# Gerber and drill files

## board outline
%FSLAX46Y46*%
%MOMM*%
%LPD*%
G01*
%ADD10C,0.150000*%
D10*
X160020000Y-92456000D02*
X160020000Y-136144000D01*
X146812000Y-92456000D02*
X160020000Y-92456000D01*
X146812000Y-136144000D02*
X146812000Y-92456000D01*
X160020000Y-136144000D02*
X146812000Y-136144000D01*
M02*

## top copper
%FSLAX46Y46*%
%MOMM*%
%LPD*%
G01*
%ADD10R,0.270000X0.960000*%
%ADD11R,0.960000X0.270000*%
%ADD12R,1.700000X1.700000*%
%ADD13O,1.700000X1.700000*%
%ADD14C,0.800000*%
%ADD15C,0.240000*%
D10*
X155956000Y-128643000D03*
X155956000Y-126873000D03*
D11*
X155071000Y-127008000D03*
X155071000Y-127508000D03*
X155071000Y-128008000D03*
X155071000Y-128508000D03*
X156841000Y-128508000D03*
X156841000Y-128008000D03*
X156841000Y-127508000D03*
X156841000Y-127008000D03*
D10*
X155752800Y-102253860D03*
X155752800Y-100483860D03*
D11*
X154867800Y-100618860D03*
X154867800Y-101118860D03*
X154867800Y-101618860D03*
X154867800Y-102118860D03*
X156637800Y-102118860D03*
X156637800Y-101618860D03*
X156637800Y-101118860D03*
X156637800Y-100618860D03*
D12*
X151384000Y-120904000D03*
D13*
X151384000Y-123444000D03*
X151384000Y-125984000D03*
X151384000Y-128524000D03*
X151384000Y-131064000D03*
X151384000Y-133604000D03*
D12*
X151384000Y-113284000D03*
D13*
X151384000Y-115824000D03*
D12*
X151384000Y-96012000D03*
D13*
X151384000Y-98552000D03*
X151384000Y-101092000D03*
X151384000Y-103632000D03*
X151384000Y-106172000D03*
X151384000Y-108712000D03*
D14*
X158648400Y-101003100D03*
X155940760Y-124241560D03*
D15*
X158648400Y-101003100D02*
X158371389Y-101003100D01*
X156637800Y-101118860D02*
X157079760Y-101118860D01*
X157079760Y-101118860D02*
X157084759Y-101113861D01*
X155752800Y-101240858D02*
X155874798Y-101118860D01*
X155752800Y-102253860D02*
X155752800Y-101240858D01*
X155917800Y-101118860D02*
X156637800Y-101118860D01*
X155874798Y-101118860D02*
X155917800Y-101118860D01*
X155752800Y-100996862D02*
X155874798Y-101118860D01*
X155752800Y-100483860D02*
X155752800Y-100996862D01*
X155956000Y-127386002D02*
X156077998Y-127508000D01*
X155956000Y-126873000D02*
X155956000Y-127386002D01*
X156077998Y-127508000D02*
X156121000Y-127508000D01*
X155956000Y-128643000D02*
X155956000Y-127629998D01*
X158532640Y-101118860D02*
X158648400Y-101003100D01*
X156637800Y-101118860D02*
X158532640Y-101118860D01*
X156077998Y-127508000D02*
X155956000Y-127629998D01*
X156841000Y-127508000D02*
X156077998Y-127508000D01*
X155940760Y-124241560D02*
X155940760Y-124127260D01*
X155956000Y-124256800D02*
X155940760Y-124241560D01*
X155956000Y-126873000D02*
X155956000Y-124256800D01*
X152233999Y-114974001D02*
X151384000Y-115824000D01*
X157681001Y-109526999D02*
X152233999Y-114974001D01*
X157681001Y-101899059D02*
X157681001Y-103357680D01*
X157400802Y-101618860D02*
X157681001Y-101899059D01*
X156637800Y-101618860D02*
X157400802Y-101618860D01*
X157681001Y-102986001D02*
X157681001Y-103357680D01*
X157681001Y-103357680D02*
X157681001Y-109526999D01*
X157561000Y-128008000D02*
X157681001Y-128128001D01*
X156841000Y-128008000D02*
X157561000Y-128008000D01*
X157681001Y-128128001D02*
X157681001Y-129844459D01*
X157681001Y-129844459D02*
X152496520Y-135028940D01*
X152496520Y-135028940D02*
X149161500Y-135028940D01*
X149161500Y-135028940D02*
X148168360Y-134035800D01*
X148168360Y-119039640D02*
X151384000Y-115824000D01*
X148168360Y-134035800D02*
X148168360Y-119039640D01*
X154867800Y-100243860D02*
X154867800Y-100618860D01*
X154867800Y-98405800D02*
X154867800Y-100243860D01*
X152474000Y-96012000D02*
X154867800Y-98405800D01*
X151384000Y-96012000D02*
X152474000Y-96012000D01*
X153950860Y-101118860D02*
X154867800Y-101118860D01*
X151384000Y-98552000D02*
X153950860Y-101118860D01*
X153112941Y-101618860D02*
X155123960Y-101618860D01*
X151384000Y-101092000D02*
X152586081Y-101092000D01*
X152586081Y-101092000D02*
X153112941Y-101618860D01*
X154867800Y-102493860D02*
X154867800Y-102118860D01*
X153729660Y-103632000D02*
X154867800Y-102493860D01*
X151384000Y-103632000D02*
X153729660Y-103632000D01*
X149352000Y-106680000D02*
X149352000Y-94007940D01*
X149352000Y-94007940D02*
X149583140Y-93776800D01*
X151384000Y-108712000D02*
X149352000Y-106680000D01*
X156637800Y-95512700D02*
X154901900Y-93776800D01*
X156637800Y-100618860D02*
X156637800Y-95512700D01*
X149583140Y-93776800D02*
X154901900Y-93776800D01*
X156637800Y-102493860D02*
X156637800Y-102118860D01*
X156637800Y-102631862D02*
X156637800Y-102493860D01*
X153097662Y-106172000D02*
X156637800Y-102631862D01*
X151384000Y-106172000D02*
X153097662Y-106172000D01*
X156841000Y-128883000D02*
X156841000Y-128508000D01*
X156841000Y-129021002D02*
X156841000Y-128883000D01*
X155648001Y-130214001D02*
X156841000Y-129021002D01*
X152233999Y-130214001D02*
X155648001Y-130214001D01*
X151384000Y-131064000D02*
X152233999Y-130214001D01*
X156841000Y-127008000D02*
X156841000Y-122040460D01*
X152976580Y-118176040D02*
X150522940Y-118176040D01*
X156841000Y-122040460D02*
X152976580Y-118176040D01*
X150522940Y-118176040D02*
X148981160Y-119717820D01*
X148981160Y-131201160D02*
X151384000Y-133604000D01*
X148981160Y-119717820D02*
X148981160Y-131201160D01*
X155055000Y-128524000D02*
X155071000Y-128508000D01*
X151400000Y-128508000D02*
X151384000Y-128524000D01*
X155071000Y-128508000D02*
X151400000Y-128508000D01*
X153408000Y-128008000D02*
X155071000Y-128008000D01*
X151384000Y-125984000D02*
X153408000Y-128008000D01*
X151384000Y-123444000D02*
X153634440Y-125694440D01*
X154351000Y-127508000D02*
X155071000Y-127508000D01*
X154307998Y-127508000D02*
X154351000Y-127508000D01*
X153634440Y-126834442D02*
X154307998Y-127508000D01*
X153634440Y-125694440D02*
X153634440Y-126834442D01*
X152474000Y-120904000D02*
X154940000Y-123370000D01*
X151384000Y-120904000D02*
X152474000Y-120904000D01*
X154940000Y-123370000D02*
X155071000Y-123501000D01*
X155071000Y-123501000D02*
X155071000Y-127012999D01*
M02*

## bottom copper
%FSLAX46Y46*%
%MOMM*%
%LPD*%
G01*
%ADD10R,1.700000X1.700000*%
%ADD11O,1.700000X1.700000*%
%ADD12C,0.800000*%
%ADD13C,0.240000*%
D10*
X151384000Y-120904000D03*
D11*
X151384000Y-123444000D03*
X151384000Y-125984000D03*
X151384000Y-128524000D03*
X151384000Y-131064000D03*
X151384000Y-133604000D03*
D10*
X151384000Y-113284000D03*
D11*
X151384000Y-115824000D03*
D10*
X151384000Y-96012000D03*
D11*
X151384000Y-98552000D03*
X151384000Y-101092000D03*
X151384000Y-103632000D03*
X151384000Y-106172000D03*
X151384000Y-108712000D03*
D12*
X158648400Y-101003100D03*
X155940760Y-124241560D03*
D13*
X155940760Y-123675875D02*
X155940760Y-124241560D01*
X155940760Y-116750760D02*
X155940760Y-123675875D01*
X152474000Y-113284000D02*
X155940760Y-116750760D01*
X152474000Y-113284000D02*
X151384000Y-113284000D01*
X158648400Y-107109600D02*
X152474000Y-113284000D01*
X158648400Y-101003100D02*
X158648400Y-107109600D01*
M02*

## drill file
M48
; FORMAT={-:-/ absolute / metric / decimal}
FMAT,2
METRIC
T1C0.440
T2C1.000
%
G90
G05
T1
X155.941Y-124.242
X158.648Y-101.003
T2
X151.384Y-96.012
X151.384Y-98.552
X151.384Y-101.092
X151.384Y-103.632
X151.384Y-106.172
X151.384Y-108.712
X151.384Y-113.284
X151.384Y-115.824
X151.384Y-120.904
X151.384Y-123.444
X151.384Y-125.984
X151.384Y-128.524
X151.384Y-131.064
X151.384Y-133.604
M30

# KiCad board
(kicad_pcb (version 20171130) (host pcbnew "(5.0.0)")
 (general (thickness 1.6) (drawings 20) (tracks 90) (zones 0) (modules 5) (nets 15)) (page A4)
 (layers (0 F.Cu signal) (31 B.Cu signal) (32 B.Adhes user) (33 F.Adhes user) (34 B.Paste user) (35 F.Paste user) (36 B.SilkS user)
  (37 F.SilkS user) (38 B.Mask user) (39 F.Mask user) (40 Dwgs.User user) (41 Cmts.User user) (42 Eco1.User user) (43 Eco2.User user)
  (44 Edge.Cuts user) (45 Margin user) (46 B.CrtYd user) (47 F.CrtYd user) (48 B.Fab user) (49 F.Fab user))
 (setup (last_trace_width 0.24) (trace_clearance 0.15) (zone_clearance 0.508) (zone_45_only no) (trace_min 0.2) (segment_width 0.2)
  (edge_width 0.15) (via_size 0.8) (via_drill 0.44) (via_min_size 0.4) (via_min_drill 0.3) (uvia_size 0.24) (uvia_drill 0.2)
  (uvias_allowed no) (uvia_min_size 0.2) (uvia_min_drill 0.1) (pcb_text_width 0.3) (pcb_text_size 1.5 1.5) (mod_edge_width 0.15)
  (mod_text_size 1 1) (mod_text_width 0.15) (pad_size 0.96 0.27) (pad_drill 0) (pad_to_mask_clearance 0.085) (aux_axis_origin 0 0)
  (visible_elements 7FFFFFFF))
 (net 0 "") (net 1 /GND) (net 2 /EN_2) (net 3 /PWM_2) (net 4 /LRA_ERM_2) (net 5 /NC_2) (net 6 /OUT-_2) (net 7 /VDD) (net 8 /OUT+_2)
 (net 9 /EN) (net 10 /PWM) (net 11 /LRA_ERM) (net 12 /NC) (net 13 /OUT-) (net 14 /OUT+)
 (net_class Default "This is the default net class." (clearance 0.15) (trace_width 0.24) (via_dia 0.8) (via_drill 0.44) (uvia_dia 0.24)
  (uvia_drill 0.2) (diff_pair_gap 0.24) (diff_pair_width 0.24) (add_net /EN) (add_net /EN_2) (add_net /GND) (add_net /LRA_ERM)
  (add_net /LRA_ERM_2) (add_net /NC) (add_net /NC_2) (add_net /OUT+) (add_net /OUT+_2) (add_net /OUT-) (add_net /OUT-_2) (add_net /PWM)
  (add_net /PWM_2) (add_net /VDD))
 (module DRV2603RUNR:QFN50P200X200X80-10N (layer F.Cu) (at 155.956 127.758)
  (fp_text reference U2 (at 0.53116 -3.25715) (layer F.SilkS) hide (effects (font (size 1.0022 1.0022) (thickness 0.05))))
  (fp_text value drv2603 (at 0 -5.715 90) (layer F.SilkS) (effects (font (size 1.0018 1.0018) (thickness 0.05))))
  (pad 5 smd rect (at 0 0.885 90) (size 0.96 0.27) (layers F.Cu F.Paste F.Mask) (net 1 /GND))
  (pad 10 smd rect (at 0 -0.885 90) (size 0.96 0.27) (layers F.Cu F.Paste F.Mask) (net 1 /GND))
  (pad 1 smd rect (at -0.885 -0.75) (size 0.96 0.27) (layers F.Cu F.Paste F.Mask) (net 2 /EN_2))
  (pad 2 smd rect (at -0.885 -0.25) (size 0.96 0.27) (layers F.Cu F.Paste F.Mask) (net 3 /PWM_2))
  (pad 3 smd rect (at -0.885 0.25) (size 0.96 0.27) (layers F.Cu F.Paste F.Mask) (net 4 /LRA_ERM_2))
  (pad 4 smd rect (at -0.885 0.75) (size 0.96 0.27) (layers F.Cu F.Paste F.Mask) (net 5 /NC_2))
  (pad 6 smd rect (at 0.885 0.75) (size 0.96 0.27) (layers F.Cu F.Paste F.Mask) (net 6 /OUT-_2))
  (pad 7 smd rect (at 0.885 0.25) (size 0.96 0.27) (layers F.Cu F.Paste F.Mask) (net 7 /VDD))
  (pad 8 smd rect (at 0.885 -0.25) (size 0.96 0.27) (layers F.Cu F.Paste F.Mask) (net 1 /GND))
  (pad 9 smd rect (at 0.885 -0.75) (size 0.96 0.27) (layers F.Cu F.Paste F.Mask) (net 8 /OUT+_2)))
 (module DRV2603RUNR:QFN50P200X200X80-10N (layer F.Cu) (at 155.7528 101.36886)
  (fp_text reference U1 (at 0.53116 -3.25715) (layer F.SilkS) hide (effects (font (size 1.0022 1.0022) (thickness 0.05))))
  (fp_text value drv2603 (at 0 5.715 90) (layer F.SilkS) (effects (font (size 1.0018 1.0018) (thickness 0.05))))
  (pad 5 smd rect (at 0 0.885 90) (size 0.96 0.27) (layers F.Cu F.Paste F.Mask) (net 1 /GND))
  (pad 10 smd rect (at 0 -0.885 90) (size 0.96 0.27) (layers F.Cu F.Paste F.Mask) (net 1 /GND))
  (pad 1 smd rect (at -0.885 -0.75) (size 0.96 0.27) (layers F.Cu F.Paste F.Mask) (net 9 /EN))
  (pad 2 smd rect (at -0.885 -0.25) (size 0.96 0.27) (layers F.Cu F.Paste F.Mask) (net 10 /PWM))
  (pad 3 smd rect (at -0.885 0.25) (size 0.96 0.27) (layers F.Cu F.Paste F.Mask) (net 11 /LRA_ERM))
  (pad 4 smd rect (at -0.885 0.75) (size 0.96 0.27) (layers F.Cu F.Paste F.Mask) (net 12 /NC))
  (pad 6 smd rect (at 0.885 0.75) (size 0.96 0.27) (layers F.Cu F.Paste F.Mask) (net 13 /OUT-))
  (pad 7 smd rect (at 0.885 0.25) (size 0.96 0.27) (layers F.Cu F.Paste F.Mask) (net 7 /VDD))
  (pad 8 smd rect (at 0.885 -0.25) (size 0.96 0.27) (layers F.Cu F.Paste F.Mask) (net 1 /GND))
  (pad 9 smd rect (at 0.885 -0.75) (size 0.96 0.27) (layers F.Cu F.Paste F.Mask) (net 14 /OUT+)))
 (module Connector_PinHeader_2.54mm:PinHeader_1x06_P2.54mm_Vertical (layer F.Cu) (at 151.384 120.904)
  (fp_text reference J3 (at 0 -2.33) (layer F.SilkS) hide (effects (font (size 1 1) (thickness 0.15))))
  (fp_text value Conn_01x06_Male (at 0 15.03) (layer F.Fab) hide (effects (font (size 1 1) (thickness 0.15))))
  (pad 1 thru_hole rect (at 0 0) (size 1.7 1.7) (drill 1) (layers *.Cu *.Mask) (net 2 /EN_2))
  (pad 2 thru_hole oval (at 0 2.54) (size 1.7 1.7) (drill 1) (layers *.Cu *.Mask) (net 3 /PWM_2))
  (pad 3 thru_hole oval (at 0 5.08) (size 1.7 1.7) (drill 1) (layers *.Cu *.Mask) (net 4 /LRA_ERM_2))
  (pad 4 thru_hole oval (at 0 7.62) (size 1.7 1.7) (drill 1) (layers *.Cu *.Mask) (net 5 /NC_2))
  (pad 5 thru_hole oval (at 0 10.16) (size 1.7 1.7) (drill 1) (layers *.Cu *.Mask) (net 6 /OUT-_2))
  (pad 6 thru_hole oval (at 0 12.7) (size 1.7 1.7) (drill 1) (layers *.Cu *.Mask) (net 8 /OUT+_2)))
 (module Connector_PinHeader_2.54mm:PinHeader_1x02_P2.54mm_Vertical (layer F.Cu) (at 151.384 113.284)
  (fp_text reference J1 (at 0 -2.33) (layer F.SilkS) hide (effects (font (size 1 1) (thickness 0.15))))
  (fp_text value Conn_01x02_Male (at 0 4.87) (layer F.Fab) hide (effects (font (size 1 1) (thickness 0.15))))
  (pad 1 thru_hole rect (at 0 0) (size 1.7 1.7) (drill 1) (layers *.Cu *.Mask) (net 1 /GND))
  (pad 2 thru_hole oval (at 0 2.54) (size 1.7 1.7) (drill 1) (layers *.Cu *.Mask) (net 7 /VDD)))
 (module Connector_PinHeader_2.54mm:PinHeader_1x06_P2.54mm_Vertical (layer F.Cu) (at 151.384 96.012)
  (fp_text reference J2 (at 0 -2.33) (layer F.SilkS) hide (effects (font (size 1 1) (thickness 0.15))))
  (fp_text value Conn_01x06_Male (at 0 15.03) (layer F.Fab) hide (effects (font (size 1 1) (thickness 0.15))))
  (pad 1 thru_hole rect (at 0 0) (size 1.7 1.7) (drill 1) (layers *.Cu *.Mask) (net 9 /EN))
  (pad 2 thru_hole oval (at 0 2.54) (size 1.7 1.7) (drill 1) (layers *.Cu *.Mask) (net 10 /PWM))
  (pad 3 thru_hole oval (at 0 5.08) (size 1.7 1.7) (drill 1) (layers *.Cu *.Mask) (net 11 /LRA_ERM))
  (pad 4 thru_hole oval (at 0 7.62) (size 1.7 1.7) (drill 1) (layers *.Cu *.Mask) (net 12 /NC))
  (pad 5 thru_hole oval (at 0 10.16) (size 1.7 1.7) (drill 1) (layers *.Cu *.Mask) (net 13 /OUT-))
  (pad 6 thru_hole oval (at 0 12.7) (size 1.7 1.7) (drill 1) (layers *.Cu *.Mask) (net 14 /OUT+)))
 (gr_line (start 160.02 92.456) (end 160.02 136.144) (layer Edge.Cuts) (width 0.15))
 (gr_line (start 146.812 92.456) (end 160.02 92.456) (layer Edge.Cuts) (width 0.15))
 (gr_line (start 146.812 136.144) (end 146.812 92.456) (layer Edge.Cuts) (width 0.15))
 (gr_line (start 160.02 136.144) (end 146.812 136.144) (layer Edge.Cuts) (width 0.15))
 (via (at 158.6484 101.0031) (size 0.8) (drill 0.44) (layers F.Cu B.Cu) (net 1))
 (segment (start 158.6484 101.0031) (end 158.371389 101.0031) (width 0.24) (layer F.Cu) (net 1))
 (segment (start 156.6378 101.11886) (end 157.07976 101.11886) (width 0.24) (layer F.Cu) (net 1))
 (segment (start 157.07976 101.11886) (end 157.084759 101.113861) (width 0.24) (layer F.Cu) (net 1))
 (segment (start 155.7528 101.240858) (end 155.874798 101.11886) (width 0.24) (layer F.Cu) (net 1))
 (segment (start 155.7528 102.25386) (end 155.7528 101.240858) (width 0.24) (layer F.Cu) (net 1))
 (segment (start 155.9178 101.11886) (end 156.6378 101.11886) (width 0.24) (layer F.Cu) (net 1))
 (segment (start 155.874798 101.11886) (end 155.9178 101.11886) (width 0.24) (layer F.Cu) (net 1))
 (segment (start 155.7528 100.996862) (end 155.874798 101.11886) (width 0.24) (layer F.Cu) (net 1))
 (segment (start 155.7528 100.48386) (end 155.7528 100.996862) (width 0.24) (layer F.Cu) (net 1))
 (segment (start 155.956 127.386002) (end 156.077998 127.508) (width 0.24) (layer F.Cu) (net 1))
 (segment (start 155.956 126.873) (end 155.956 127.386002) (width 0.24) (layer F.Cu) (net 1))
 (segment (start 156.077998 127.508) (end 156.121 127.508) (width 0.24) (layer F.Cu) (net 1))
 (segment (start 155.956 128.643) (end 155.956 127.629998) (width 0.24) (layer F.Cu) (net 1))
 (segment (start 158.53264 101.11886) (end 158.6484 101.0031) (width 0.24) (layer F.Cu) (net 1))
 (segment (start 156.6378 101.11886) (end 158.53264 101.11886) (width 0.24) (layer F.Cu) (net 1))
 (segment (start 156.077998 127.508) (end 155.956 127.629998) (width 0.24) (layer F.Cu) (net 1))
 (segment (start 156.841 127.508) (end 156.077998 127.508) (width 0.24) (layer F.Cu) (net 1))
 (segment (start 155.94076 124.24156) (end 155.94076 124.12726) (width 0.24) (layer F.Cu) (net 1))
 (via (at 155.94076 124.24156) (size 0.8) (drill 0.44) (layers F.Cu B.Cu) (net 1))
 (segment (start 155.94076 123.675875) (end 155.94076 124.24156) (width 0.24) (layer B.Cu) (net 1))
 (segment (start 155.94076 116.75076) (end 155.94076 123.675875) (width 0.24) (layer B.Cu) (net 1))
 (segment (start 152.474 113.284) (end 155.94076 116.75076) (width 0.24) (layer B.Cu) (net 1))
 (segment (start 155.956 124.2568) (end 155.94076 124.24156) (width 0.24) (layer F.Cu) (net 1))
 (segment (start 155.956 126.873) (end 155.956 124.2568) (width 0.24) (layer F.Cu) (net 1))
 (segment (start 152.474 113.284) (end 151.384 113.284) (width 0.24) (layer B.Cu) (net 1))
 (segment (start 158.6484 107.1096) (end 152.474 113.284) (width 0.24) (layer B.Cu) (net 1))
 (segment (start 158.6484 101.0031) (end 158.6484 107.1096) (width 0.24) (layer B.Cu) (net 1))
 (segment (start 152.233999 114.974001) (end 151.384 115.824) (width 0.24) (layer F.Cu) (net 7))
 (segment (start 157.681001 109.526999) (end 152.233999 114.974001) (width 0.24) (layer F.Cu) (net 7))
 (segment (start 157.681001 101.899059) (end 157.681001 103.35768) (width 0.24) (layer F.Cu) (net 7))
 (segment (start 157.400802 101.61886) (end 157.681001 101.899059) (width 0.24) (layer F.Cu) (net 7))
 (segment (start 156.6378 101.61886) (end 157.400802 101.61886) (width 0.24) (layer F.Cu) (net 7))
 (segment (start 157.681001 102.986001) (end 157.681001 103.35768) (width 0.24) (layer F.Cu) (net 7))
 (segment (start 157.681001 103.35768) (end 157.681001 109.526999) (width 0.24) (layer F.Cu) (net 7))
 (segment (start 157.561 128.008) (end 157.681001 128.128001) (width 0.24) (layer F.Cu) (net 7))
 (segment (start 156.841 128.008) (end 157.561 128.008) (width 0.24) (layer F.Cu) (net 7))
 (segment (start 157.681001 128.128001) (end 157.681001 129.844459) (width 0.24) (layer F.Cu) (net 7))
 (segment (start 157.681001 129.844459) (end 152.49652 135.02894) (width 0.24) (layer F.Cu) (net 7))
 (segment (start 152.49652 135.02894) (end 149.1615 135.02894) (width 0.24) (layer F.Cu) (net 7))
 (segment (start 149.1615 135.02894) (end 148.16836 134.0358) (width 0.24) (layer F.Cu) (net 7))
 (segment (start 148.16836 119.03964) (end 151.384 115.824) (width 0.24) (layer F.Cu) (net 7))
 (segment (start 148.16836 134.0358) (end 148.16836 119.03964) (width 0.24) (layer F.Cu) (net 7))
 (segment (start 154.8678 100.24386) (end 154.8678 100.61886) (width 0.24) (layer F.Cu) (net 9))
 (segment (start 154.8678 98.4058) (end 154.8678 100.24386) (width 0.24) (layer F.Cu) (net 9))
 (segment (start 152.474 96.012) (end 154.8678 98.4058) (width 0.24) (layer F.Cu) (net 9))
 (segment (start 151.384 96.012) (end 152.474 96.012) (width 0.24) (layer F.Cu) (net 9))
 (segment (start 153.95086 101.11886) (end 154.8678 101.11886) (width 0.24) (layer F.Cu) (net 10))
 (segment (start 151.384 98.552) (end 153.95086 101.11886) (width 0.24) (layer F.Cu) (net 10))
 (segment (start 153.112941 101.61886) (end 155.12396 101.61886) (width 0.24) (layer F.Cu) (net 11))
 (segment (start 151.384 101.092) (end 152.586081 101.092) (width 0.24) (layer F.Cu) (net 11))
 (segment (start 152.586081 101.092) (end 153.112941 101.61886) (width 0.24) (layer F.Cu) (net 11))
 (segment (start 154.8678 102.49386) (end 154.8678 102.11886) (width 0.24) (layer F.Cu) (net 12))
 (segment (start 153.72966 103.632) (end 154.8678 102.49386) (width 0.24) (layer F.Cu) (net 12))
 (segment (start 151.384 103.632) (end 153.72966 103.632) (width 0.24) (layer F.Cu) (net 12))
 (segment (start 149.352 106.68) (end 149.352 94.00794) (width 0.24) (layer F.Cu) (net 14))
 (segment (start 149.352 94.00794) (end 149.58314 93.7768) (width 0.24) (layer F.Cu) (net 14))
 (segment (start 151.384 108.712) (end 149.352 106.68) (width 0.24) (layer F.Cu) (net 14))
 (segment (start 156.6378 95.5127) (end 154.9019 93.7768) (width 0.24) (layer F.Cu) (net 14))
 (segment (start 156.6378 100.61886) (end 156.6378 95.5127) (width 0.24) (layer F.Cu) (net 14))
 (segment (start 149.58314 93.7768) (end 154.9019 93.7768) (width 0.24) (layer F.Cu) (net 14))
 (segment (start 156.6378 102.49386) (end 156.6378 102.11886) (width 0.24) (layer F.Cu) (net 13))
 (segment (start 156.6378 102.631862) (end 156.6378 102.49386) (width 0.24) (layer F.Cu) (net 13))
 (segment (start 153.097662 106.172) (end 156.6378 102.631862) (width 0.24) (layer F.Cu) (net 13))
 (segment (start 151.384 106.172) (end 153.097662 106.172) (width 0.24) (layer F.Cu) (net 13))
 (segment (start 156.841 128.883) (end 156.841 128.508) (width 0.24) (layer F.Cu) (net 6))
 (segment (start 156.841 129.021002) (end 156.841 128.883) (width 0.24) (layer F.Cu) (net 6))
 (segment (start 155.648001 130.214001) (end 156.841 129.021002) (width 0.24) (layer F.Cu) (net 6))
 (segment (start 152.233999 130.214001) (end 155.648001 130.214001) (width 0.24) (layer F.Cu) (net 6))
 (segment (start 151.384 131.064) (end 152.233999 130.214001) (width 0.24) (layer F.Cu) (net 6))
 (segment (start 156.841 127.008) (end 156.841 122.04046) (width 0.24) (layer F.Cu) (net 8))
 (segment (start 152.97658 118.17604) (end 150.52294 118.17604) (width 0.24) (layer F.Cu) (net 8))
 (segment (start 156.841 122.04046) (end 152.97658 118.17604) (width 0.24) (layer F.Cu) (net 8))
 (segment (start 150.52294 118.17604) (end 148.98116 119.71782) (width 0.24) (layer F.Cu) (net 8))
 (segment (start 148.98116 131.20116) (end 151.384 133.604) (width 0.24) (layer F.Cu) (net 8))
 (segment (start 148.98116 119.71782) (end 148.98116 131.20116) (width 0.24) (layer F.Cu) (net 8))
 (segment (start 155.055 128.524) (end 155.071 128.508) (width 0.24) (layer F.Cu) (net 5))
 (segment (start 151.4 128.508) (end 151.384 128.524) (width 0.24) (layer F.Cu) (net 5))
 (segment (start 155.071 128.508) (end 151.4 128.508) (width 0.24) (layer F.Cu) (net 5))
 (segment (start 153.408 128.008) (end 155.071 128.008) (width 0.24) (layer F.Cu) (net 4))
 (segment (start 151.384 125.984) (end 153.408 128.008) (width 0.24) (layer F.Cu) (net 4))
 (segment (start 151.384 123.444) (end 153.63444 125.69444) (width 0.24) (layer F.Cu) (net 3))
 (segment (start 154.351 127.508) (end 155.071 127.508) (width 0.24) (layer F.Cu) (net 3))
 (segment (start 154.307998 127.508) (end 154.351 127.508) (width 0.24) (layer F.Cu) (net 3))
 (segment (start 153.63444 126.834442) (end 154.307998 127.508) (width 0.24) (layer F.Cu) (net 3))
 (segment (start 153.63444 125.69444) (end 153.63444 126.834442) (width 0.24) (layer F.Cu) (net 3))
 (segment (start 152.474 120.904) (end 154.94 123.37) (width 0.24) (layer F.Cu) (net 2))
 (segment (start 151.384 120.904) (end 152.474 120.904) (width 0.24) (layer F.Cu) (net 2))
 (segment (start 154.94 123.37) (end 155.071 123.501) (width 0.24) (layer F.Cu) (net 2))
 (segment (start 155.071 123.501) (end 155.071 127.012999) (width 0.24) (layer F.Cu) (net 2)))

